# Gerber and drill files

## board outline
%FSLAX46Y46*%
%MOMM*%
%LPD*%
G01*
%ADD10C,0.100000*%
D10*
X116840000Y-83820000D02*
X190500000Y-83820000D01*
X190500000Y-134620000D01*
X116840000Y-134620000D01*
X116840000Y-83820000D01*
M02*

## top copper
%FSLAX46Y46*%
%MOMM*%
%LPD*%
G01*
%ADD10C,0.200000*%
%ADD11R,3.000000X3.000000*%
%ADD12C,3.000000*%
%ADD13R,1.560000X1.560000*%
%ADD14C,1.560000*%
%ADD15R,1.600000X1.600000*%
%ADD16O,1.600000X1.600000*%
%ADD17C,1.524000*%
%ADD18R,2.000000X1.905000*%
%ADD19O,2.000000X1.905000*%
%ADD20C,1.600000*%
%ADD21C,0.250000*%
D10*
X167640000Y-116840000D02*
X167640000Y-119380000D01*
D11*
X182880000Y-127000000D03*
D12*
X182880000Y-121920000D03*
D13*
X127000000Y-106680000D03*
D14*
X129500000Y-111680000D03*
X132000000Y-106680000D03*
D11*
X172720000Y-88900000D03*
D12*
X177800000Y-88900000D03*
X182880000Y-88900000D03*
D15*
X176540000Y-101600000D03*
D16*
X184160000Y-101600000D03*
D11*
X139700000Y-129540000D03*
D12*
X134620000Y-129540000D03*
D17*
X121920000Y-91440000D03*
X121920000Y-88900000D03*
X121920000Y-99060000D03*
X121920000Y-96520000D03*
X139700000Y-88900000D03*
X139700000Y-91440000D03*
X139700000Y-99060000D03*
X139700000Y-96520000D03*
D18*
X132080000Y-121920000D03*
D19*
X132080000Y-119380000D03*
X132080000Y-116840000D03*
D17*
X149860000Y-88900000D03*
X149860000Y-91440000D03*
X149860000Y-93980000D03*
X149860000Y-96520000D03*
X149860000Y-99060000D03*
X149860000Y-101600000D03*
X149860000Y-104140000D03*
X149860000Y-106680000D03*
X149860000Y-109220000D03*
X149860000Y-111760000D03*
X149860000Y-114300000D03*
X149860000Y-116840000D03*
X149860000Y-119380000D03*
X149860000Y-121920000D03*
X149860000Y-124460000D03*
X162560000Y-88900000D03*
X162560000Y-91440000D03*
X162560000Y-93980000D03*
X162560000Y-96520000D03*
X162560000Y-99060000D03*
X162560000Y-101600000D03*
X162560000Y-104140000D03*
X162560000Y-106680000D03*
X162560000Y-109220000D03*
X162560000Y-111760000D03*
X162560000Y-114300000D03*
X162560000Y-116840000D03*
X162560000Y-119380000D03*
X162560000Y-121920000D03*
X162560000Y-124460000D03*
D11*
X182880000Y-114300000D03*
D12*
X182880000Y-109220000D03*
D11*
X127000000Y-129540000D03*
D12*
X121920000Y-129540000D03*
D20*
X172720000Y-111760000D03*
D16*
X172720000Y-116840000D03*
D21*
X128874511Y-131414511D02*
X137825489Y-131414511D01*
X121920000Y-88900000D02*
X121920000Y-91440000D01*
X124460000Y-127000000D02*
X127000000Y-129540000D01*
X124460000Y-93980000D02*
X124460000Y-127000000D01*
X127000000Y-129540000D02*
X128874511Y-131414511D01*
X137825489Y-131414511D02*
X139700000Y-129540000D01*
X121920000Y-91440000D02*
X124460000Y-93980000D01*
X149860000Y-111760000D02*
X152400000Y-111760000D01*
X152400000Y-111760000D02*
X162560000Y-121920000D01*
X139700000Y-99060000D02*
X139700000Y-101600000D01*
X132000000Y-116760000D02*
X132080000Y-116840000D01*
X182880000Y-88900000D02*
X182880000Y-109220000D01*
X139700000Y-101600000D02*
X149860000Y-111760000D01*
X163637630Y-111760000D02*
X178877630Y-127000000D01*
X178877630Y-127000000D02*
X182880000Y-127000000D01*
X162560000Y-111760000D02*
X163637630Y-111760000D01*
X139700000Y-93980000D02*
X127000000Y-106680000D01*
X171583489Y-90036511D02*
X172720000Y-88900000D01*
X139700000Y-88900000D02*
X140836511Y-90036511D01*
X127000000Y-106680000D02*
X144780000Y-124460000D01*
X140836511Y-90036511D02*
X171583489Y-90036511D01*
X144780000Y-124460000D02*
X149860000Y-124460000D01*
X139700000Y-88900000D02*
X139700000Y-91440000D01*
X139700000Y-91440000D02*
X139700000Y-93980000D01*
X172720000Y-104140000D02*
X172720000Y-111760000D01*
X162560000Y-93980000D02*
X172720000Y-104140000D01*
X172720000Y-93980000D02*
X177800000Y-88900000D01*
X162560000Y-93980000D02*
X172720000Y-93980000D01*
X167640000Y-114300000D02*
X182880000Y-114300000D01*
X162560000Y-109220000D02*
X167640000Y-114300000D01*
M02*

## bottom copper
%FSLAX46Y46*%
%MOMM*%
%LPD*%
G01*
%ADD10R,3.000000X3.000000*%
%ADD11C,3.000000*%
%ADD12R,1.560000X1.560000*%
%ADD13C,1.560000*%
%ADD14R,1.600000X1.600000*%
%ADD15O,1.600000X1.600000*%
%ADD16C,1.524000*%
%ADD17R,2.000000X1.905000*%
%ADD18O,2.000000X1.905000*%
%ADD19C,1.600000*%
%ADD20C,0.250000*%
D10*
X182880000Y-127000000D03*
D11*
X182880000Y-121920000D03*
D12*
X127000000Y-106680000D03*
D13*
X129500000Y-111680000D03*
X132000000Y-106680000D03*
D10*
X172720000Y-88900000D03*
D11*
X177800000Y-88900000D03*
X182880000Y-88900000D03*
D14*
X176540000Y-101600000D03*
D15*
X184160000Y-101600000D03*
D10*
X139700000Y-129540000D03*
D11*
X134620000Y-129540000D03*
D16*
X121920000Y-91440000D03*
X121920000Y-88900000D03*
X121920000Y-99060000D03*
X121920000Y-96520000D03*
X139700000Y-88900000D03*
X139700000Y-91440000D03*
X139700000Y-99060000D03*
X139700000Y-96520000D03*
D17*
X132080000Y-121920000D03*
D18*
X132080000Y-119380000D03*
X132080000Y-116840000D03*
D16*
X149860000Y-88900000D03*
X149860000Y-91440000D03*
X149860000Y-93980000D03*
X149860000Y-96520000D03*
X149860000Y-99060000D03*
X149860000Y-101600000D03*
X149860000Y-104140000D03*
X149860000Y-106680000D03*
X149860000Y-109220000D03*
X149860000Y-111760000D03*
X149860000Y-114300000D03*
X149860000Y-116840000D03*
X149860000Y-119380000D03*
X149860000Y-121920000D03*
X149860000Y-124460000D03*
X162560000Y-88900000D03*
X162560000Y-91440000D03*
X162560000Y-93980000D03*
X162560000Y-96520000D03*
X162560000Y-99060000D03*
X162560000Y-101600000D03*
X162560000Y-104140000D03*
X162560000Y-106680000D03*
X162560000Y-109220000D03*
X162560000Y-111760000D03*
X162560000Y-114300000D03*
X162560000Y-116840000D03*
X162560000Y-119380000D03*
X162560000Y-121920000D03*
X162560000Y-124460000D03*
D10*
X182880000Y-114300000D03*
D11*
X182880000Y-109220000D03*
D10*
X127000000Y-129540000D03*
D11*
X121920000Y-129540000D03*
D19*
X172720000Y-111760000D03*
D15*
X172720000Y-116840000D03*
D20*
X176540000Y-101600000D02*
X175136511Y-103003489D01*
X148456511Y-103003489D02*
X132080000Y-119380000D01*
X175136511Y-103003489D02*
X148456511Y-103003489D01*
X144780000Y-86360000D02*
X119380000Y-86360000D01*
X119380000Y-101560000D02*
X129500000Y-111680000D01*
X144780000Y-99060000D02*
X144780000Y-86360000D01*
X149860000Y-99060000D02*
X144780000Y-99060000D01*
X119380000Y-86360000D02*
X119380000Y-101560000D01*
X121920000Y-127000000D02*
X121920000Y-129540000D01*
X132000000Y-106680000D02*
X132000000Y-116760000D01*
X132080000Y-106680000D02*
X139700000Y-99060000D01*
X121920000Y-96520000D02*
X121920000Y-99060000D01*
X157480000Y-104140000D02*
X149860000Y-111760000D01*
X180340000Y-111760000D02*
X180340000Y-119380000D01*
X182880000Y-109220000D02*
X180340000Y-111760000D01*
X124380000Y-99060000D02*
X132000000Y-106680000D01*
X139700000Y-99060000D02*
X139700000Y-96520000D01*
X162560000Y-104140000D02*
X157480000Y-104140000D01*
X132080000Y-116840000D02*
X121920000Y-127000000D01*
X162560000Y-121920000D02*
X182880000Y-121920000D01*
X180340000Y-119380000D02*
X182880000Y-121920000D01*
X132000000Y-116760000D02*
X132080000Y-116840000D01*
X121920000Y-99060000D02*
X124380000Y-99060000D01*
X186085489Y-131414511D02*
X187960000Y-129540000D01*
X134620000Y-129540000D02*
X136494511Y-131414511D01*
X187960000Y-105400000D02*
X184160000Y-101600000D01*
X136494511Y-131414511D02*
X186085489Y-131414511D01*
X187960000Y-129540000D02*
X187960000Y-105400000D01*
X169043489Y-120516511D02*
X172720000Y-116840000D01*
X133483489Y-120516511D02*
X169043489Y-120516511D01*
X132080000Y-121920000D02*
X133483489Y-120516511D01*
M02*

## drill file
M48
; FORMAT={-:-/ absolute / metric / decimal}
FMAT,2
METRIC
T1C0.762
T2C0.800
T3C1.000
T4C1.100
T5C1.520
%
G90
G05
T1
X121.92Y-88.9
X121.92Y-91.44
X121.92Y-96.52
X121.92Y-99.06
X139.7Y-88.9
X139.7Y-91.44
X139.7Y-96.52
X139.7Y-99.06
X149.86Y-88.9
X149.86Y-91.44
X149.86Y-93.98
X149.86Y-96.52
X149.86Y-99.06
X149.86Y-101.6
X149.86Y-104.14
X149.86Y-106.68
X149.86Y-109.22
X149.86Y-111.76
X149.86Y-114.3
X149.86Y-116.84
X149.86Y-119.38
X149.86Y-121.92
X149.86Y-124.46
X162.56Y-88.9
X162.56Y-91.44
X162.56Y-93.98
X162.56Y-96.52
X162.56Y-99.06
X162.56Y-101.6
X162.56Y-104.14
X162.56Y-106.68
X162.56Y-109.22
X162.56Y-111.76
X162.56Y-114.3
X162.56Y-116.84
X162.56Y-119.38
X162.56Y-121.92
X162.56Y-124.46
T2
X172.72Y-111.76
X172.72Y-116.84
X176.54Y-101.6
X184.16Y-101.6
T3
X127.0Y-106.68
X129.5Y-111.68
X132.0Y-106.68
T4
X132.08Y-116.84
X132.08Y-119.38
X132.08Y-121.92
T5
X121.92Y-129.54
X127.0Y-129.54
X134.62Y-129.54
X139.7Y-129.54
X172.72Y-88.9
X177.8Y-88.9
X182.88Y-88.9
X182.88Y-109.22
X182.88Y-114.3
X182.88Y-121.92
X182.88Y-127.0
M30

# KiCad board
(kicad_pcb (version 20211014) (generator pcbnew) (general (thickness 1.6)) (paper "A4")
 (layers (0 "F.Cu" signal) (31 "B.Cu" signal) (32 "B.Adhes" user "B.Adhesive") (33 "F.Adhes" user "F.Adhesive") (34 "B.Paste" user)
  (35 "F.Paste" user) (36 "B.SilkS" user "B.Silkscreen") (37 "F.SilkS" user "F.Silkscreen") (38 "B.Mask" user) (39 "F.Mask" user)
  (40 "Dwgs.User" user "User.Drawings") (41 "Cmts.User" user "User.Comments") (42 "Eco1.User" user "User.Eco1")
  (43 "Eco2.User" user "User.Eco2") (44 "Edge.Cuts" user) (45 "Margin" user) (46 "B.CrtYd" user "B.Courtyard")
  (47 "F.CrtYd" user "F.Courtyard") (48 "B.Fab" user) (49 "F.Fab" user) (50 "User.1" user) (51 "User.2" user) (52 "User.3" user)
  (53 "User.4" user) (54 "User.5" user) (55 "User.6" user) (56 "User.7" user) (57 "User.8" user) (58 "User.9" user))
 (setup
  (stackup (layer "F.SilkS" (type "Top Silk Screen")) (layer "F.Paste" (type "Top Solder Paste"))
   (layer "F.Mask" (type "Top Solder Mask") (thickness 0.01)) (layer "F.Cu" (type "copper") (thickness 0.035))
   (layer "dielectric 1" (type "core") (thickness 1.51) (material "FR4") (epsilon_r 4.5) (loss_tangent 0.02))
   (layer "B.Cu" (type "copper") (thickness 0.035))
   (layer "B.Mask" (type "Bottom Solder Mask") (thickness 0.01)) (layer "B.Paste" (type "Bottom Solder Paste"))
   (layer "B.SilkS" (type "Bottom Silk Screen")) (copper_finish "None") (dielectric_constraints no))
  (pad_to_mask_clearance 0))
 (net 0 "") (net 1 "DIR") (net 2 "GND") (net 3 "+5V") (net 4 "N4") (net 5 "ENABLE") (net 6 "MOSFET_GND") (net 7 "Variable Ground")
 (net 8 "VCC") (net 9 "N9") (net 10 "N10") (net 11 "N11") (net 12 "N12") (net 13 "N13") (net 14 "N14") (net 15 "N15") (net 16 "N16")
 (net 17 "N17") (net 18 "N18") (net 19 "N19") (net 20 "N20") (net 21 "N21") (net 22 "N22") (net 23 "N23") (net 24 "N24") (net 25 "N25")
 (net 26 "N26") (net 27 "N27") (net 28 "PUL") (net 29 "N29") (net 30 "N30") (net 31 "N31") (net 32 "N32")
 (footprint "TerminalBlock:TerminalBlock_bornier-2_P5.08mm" (layer "F.Cu") (at 182.88 127 90)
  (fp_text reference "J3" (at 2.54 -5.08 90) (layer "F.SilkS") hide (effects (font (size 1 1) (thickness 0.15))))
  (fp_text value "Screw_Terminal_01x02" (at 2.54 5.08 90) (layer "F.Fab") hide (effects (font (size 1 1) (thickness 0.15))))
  (pad "1" thru_hole rect (at 0 0 90) (size 3 3) (drill 1.52) (layers *.Cu *.Mask) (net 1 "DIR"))
  (pad "2" thru_hole circle (at 5.08 0 90) (size 3 3) (drill 1.52) (layers *.Cu *.Mask) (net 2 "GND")))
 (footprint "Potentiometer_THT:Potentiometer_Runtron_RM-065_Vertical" (layer "F.Cu") (at 127 106.68)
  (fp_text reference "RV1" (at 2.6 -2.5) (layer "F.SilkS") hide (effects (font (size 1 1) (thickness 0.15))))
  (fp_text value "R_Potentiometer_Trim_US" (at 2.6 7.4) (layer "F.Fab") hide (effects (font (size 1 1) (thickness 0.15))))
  (pad "1" thru_hole rect (at 0 0) (size 1.56 1.56) (drill 1) (layers *.Cu *.Mask) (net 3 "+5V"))
  (pad "2" thru_hole circle (at 2.5 5) (size 1.56 1.56) (drill 1) (layers *.Cu *.Mask) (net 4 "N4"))
  (pad "3" thru_hole circle (at 5 0) (size 1.56 1.56) (drill 1) (layers *.Cu *.Mask) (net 2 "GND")))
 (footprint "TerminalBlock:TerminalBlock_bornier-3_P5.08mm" (layer "F.Cu") (at 172.72 88.9)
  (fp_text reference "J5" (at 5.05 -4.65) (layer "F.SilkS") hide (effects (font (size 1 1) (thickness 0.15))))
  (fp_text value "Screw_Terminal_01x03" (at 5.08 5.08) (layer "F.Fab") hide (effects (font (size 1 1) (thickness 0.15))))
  (pad "1" thru_hole rect (at 0 0) (size 3 3) (drill 1.52) (layers *.Cu *.Mask) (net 3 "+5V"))
  (pad "2" thru_hole circle (at 5.08 0) (size 3 3) (drill 1.52) (layers *.Cu *.Mask) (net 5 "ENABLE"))
  (pad "3" thru_hole circle (at 10.16 0) (size 3 3) (drill 1.52) (layers *.Cu *.Mask) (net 2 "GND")))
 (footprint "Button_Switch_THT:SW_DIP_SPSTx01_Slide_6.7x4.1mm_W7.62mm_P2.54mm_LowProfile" (layer "F.Cu") (at 176.54 101.6)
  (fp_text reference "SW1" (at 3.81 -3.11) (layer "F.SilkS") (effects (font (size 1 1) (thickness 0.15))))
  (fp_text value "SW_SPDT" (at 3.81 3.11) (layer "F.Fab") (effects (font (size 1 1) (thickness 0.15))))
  (pad "1" thru_hole rect (at 0 0) (size 1.6 1.6) (drill 0.8) (layers *.Cu *.Mask) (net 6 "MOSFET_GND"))
  (pad "2" thru_hole oval (at 7.62 0) (size 1.6 1.6) (drill 0.8) (layers *.Cu *.Mask) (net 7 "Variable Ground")))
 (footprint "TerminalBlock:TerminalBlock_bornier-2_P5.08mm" (layer "F.Cu") (at 139.7 129.54 180)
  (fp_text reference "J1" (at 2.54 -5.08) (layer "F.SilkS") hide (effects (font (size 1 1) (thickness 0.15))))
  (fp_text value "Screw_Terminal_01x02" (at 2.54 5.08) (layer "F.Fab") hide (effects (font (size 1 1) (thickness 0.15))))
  (pad "1" thru_hole rect (at 0 0 180) (size 3 3) (drill 1.52) (layers *.Cu *.Mask) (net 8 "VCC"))
  (pad "2" thru_hole circle (at 5.08 0 180) (size 3 3) (drill 1.52) (layers *.Cu *.Mask) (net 7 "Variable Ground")))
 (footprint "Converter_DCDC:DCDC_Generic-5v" (layer "F.Cu") (at 132.08 96.52)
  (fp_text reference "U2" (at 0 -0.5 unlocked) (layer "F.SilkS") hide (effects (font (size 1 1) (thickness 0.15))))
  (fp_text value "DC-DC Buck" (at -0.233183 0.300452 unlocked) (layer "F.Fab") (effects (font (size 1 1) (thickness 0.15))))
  (pad "1" thru_hole circle (at -10.16 -5.08) (size 1.524 1.524) (drill 0.762) (layers *.Cu *.Mask) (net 8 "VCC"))
  (pad "1" thru_hole circle (at -10.16 -7.62) (size 1.524 1.524) (drill 0.762) (layers *.Cu *.Mask) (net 8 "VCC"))
  (pad "2" thru_hole circle (at -10.16 2.54) (size 1.524 1.524) (drill 0.762) (layers *.Cu *.Mask) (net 2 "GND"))
  (pad "2" thru_hole circle (at -10.16 0) (size 1.524 1.524) (drill 0.762) (layers *.Cu *.Mask) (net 2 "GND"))
  (pad "3" thru_hole circle (at 7.62 -7.62) (size 1.524 1.524) (drill 0.762) (layers *.Cu *.Mask) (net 3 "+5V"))
  (pad "3" thru_hole circle (at 7.62 -5.08) (size 1.524 1.524) (drill 0.762) (layers *.Cu *.Mask) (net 3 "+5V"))
  (pad "4" thru_hole circle (at 7.62 2.54) (size 1.524 1.524) (drill 0.762) (layers *.Cu *.Mask) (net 2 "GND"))
  (pad "4" thru_hole circle (at 7.62 0) (size 1.524 1.524) (drill 0.762) (layers *.Cu *.Mask) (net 2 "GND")))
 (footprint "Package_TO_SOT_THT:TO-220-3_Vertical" (layer "F.Cu") (at 132.08 121.92 90)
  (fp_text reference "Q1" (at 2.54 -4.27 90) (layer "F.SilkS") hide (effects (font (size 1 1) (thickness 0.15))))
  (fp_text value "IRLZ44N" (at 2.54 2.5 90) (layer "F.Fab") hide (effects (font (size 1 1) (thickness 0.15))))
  (pad "1" thru_hole rect (at 0 0 90) (size 1.905 2) (drill 1.1) (layers *.Cu *.Mask) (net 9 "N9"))
  (pad "2" thru_hole oval (at 2.54 0 90) (size 1.905 2) (drill 1.1) (layers *.Cu *.Mask) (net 6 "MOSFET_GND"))
  (pad "3" thru_hole oval (at 5.08 0 90) (size 1.905 2) (drill 1.1) (layers *.Cu *.Mask) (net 2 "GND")))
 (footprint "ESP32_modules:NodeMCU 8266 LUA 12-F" (layer "F.Cu") (at 154.94 99.06)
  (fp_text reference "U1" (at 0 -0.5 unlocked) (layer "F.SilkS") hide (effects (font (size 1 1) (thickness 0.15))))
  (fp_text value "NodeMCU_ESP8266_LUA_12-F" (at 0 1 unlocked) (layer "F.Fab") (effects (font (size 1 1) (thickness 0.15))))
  (pad "1" thru_hole circle (at -5.08 -10.16) (size 1.524 1.524) (drill 0.762) (layers *.Cu *.Mask) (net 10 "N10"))
  (pad "2" thru_hole circle (at -5.08 -7.62) (size 1.524 1.524) (drill 0.762) (layers *.Cu *.Mask) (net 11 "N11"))
  (pad "3" thru_hole circle (at -5.08 -5.08) (size 1.524 1.524) (drill 0.762) (layers *.Cu *.Mask) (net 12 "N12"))
  (pad "4" thru_hole circle (at -5.08 -2.54) (size 1.524 1.524) (drill 0.762) (layers *.Cu *.Mask) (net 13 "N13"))
  (pad "5" thru_hole circle (at -5.08 0) (size 1.524 1.524) (drill 0.762) (layers *.Cu *.Mask) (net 4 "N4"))
  (pad "6" thru_hole circle (at -5.08 2.54) (size 1.524 1.524) (drill 0.762) (layers *.Cu *.Mask) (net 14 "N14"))
  (pad "7" thru_hole circle (at -5.08 5.08) (size 1.524 1.524) (drill 0.762) (layers *.Cu *.Mask) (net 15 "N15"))
  (pad "8" thru_hole circle (at -5.08 7.62) (size 1.524 1.524) (drill 0.762) (layers *.Cu *.Mask) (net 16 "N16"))
  (pad "9" thru_hole circle (at -5.08 10.16) (size 1.524 1.524) (drill 0.762) (layers *.Cu *.Mask) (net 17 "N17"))
  (pad "10" thru_hole circle (at -5.08 12.7) (size 1.524 1.524) (drill 0.762) (layers *.Cu *.Mask) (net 2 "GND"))
  (pad "11" thru_hole circle (at -5.08 15.24) (size 1.524 1.524) (drill 0.762) (layers *.Cu *.Mask) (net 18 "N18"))
  (pad "12" thru_hole circle (at -5.08 17.78) (size 1.524 1.524) (drill 0.762) (layers *.Cu *.Mask) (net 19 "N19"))
  (pad "13" thru_hole circle (at -5.08 20.32) (size 1.524 1.524) (drill 0.762) (layers *.Cu *.Mask) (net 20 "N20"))
  (pad "14" thru_hole circle (at -5.08 22.86) (size 1.524 1.524) (drill 0.762) (layers *.Cu *.Mask) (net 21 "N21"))
  (pad "15" thru_hole circle (at -5.08 25.4) (size 1.524 1.524) (drill 0.762) (layers *.Cu *.Mask) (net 3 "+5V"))
  (pad "16" thru_hole circle (at 7.62 -10.16) (size 1.524 1.524) (drill 0.762) (layers *.Cu *.Mask) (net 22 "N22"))
  (pad "17" thru_hole circle (at 7.62 -7.62) (size 1.524 1.524) (drill 0.762) (layers *.Cu *.Mask) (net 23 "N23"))
  (pad "18" thru_hole circle (at 7.62 -5.08) (size 1.524 1.524) (drill 0.762) (layers *.Cu *.Mask) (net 5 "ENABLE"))
  (pad "19" thru_hole circle (at 7.62 -2.54) (size 1.524 1.524) (drill 0.762) (layers *.Cu *.Mask) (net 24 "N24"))
  (pad "20" thru_hole circle (at 7.62 0) (size 1.524 1.524) (drill 0.762) (layers *.Cu *.Mask) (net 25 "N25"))
  (pad "21" thru_hole circle (at 7.62 2.54) (size 1.524 1.524) (drill 0.762) (layers *.Cu *.Mask) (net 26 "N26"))
  (pad "22" thru_hole circle (at 7.62 5.08) (size 1.524 1.524) (drill 0.762) (layers *.Cu *.Mask) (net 2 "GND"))
  (pad "23" thru_hole circle (at 7.62 7.62) (size 1.524 1.524) (drill 0.762) (layers *.Cu *.Mask) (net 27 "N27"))
  (pad "24" thru_hole circle (at 7.62 10.16) (size 1.524 1.524) (drill 0.762) (layers *.Cu *.Mask) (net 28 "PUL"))
  (pad "25" thru_hole circle (at 7.62 12.7) (size 1.524 1.524) (drill 0.762) (layers *.Cu *.Mask) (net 1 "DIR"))
  (pad "26" thru_hole circle (at 7.62 15.24) (size 1.524 1.524) (drill 0.762) (layers *.Cu *.Mask) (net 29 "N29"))
  (pad "27" thru_hole circle (at 7.62 17.78) (size 1.524 1.524) (drill 0.762) (layers *.Cu *.Mask) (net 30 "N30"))
  (pad "28" thru_hole circle (at 7.62 20.32) (size 1.524 1.524) (drill 0.762) (layers *.Cu *.Mask) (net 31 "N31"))
  (pad "29" thru_hole circle (at 7.62 22.86) (size 1.524 1.524) (drill 0.762) (layers *.Cu *.Mask) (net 2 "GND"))
  (pad "30" thru_hole circle (at 7.62 25.4) (size 1.524 1.524) (drill 0.762) (layers *.Cu *.Mask) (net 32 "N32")))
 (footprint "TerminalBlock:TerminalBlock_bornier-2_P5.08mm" (layer "F.Cu") (at 182.88 114.3 90)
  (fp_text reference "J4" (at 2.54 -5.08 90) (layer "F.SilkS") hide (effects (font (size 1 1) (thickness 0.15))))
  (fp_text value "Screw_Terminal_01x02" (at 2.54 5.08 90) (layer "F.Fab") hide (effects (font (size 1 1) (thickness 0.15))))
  (pad "1" thru_hole rect (at 0 0 90) (size 3 3) (drill 1.52) (layers *.Cu *.Mask) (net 28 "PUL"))
  (pad "2" thru_hole circle (at 5.08 0 90) (size 3 3) (drill 1.52) (layers *.Cu *.Mask) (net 2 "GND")))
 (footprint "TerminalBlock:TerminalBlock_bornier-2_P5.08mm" (layer "F.Cu") (at 127 129.54 180)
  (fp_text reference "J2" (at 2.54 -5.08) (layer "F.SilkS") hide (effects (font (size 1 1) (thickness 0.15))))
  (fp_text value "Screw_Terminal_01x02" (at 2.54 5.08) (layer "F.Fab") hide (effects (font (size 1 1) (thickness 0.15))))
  (pad "1" thru_hole rect (at 0 0 180) (size 3 3) (drill 1.52) (layers *.Cu *.Mask) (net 8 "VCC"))
  (pad "2" thru_hole circle (at 5.08 0 180) (size 3 3) (drill 1.52) (layers *.Cu *.Mask) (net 2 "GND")))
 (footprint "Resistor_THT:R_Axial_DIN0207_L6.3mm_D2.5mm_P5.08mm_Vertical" (layer "F.Cu") (at 172.72 111.76 -90)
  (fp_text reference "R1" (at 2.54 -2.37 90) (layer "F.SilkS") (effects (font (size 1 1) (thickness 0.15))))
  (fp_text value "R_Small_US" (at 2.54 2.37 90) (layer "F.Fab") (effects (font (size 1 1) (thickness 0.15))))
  (pad "1" thru_hole circle (at 0 0 270) (size 1.6 1.6) (drill 0.8) (layers *.Cu *.Mask) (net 5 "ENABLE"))
  (pad "2" thru_hole oval (at 5.08 0 270) (size 1.6 1.6) (drill 0.8) (layers *.Cu *.Mask) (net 9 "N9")))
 (gr_line (start 167.64 116.84) (end 167.64 119.38) (layer "F.Cu") (width 0.2))
 (gr_rect (start 116.84 83.82) (end 190.5 134.62) (layer "Edge.Cuts") (width 0.1) (fill none))
 (segment (start 128.874511 131.414511) (end 137.825489 131.414511) (width 0.25) (layer "F.Cu") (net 8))
 (segment (start 121.92 88.9) (end 121.92 91.44) (width 0.25) (layer "F.Cu") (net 8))
 (segment (start 124.46 127) (end 127 129.54) (width 0.25) (layer "F.Cu") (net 8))
 (segment (start 124.46 93.98) (end 124.46 127) (width 0.25) (layer "F.Cu") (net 8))
 (segment (start 127 129.54) (end 128.874511 131.414511) (width 0.25) (layer "F.Cu") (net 8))
 (segment (start 137.825489 131.414511) (end 139.7 129.54) (width 0.25) (layer "F.Cu") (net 8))
 (segment (start 121.92 91.44) (end 124.46 93.98) (width 0.25) (layer "F.Cu") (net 8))
 (segment (start 176.54 101.6) (end 175.136511 103.003489) (width 0.25) (layer "B.Cu") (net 6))
 (segment (start 148.456511 103.003489) (end 132.08 119.38) (width 0.25) (layer "B.Cu") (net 6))
 (segment (start 175.136511 103.003489) (end 148.456511 103.003489) (width 0.25) (layer "B.Cu") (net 6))
 (segment (start 144.78 86.36) (end 119.38 86.36) (width 0.25) (layer "B.Cu") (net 4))
 (segment (start 119.38 101.56) (end 129.5 111.68) (width 0.25) (layer "B.Cu") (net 4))
 (segment (start 144.78 99.06) (end 144.78 86.36) (width 0.25) (layer "B.Cu") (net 4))
 (segment (start 149.86 99.06) (end 144.78 99.06) (width 0.25) (layer "B.Cu") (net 4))
 (segment (start 119.38 86.36) (end 119.38 101.56) (width 0.25) (layer "B.Cu") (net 4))
 (segment (start 149.86 111.76) (end 152.4 111.76) (width 0.25) (layer "F.Cu") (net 2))
 (segment (start 152.4 111.76) (end 162.56 121.92) (width 0.25) (layer "F.Cu") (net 2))
 (segment (start 139.7 99.06) (end 139.7 101.6) (width 0.25) (layer "F.Cu") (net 2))
 (segment (start 132 116.76) (end 132.08 116.84) (width 0.25) (layer "F.Cu") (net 2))
 (segment (start 182.88 88.9) (end 182.88 109.22) (width 0.25) (layer "F.Cu") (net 2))
 (segment (start 139.7 101.6) (end 149.86 111.76) (width 0.25) (layer "F.Cu") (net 2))
 (segment (start 121.92 127) (end 121.92 129.54) (width 0.25) (layer "B.Cu") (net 2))
 (segment (start 132 106.68) (end 132 116.76) (width 0.25) (layer "B.Cu") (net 2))
 (segment (start 132.08 106.68) (end 139.7 99.06) (width 0.25) (layer "B.Cu") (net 2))
 (segment (start 121.92 96.52) (end 121.92 99.06) (width 0.25) (layer "B.Cu") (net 2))
 (segment (start 157.48 104.14) (end 149.86 111.76) (width 0.25) (layer "B.Cu") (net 2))
 (segment (start 180.34 111.76) (end 180.34 119.38) (width 0.25) (layer "B.Cu") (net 2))
 (segment (start 182.88 109.22) (end 180.34 111.76) (width 0.25) (layer "B.Cu") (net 2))
 (segment (start 124.38 99.06) (end 132 106.68) (width 0.25) (layer "B.Cu") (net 2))
 (segment (start 139.7 99.06) (end 139.7 96.52) (width 0.25) (layer "B.Cu") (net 2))
 (segment (start 162.56 104.14) (end 157.48 104.14) (width 0.25) (layer "B.Cu") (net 2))
 (segment (start 132.08 116.84) (end 121.92 127) (width 0.25) (layer "B.Cu") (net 2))
 (segment (start 162.56 121.92) (end 182.88 121.92) (width 0.25) (layer "B.Cu") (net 2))
 (segment (start 180.34 119.38) (end 182.88 121.92) (width 0.25) (layer "B.Cu") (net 2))
 (segment (start 132 116.76) (end 132.08 116.84) (width 0.25) (layer "B.Cu") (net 2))
 (segment (start 121.92 99.06) (end 124.38 99.06) (width 0.25) (layer "B.Cu") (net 2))
 (segment (start 186.085489 131.414511) (end 187.96 129.54) (width 0.25) (layer "B.Cu") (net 7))
 (segment (start 134.62 129.54) (end 136.494511 131.414511) (width 0.25) (layer "B.Cu") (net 7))
 (segment (start 187.96 105.4) (end 184.16 101.6) (width 0.25) (layer "B.Cu") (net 7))
 (segment (start 136.494511 131.414511) (end 186.085489 131.414511) (width 0.25) (layer "B.Cu") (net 7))
 (segment (start 187.96 129.54) (end 187.96 105.4) (width 0.25) (layer "B.Cu") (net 7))
 (segment (start 163.63763 111.76) (end 178.87763 127) (width 0.25) (layer "F.Cu") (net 1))
 (segment (start 178.87763 127) (end 182.88 127) (width 0.25) (layer "F.Cu") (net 1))
 (segment (start 162.56 111.76) (end 163.63763 111.76) (width 0.25) (layer "F.Cu") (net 1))
 (segment (start 139.7 93.98) (end 127 106.68) (width 0.25) (layer "F.Cu") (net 3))
 (segment (start 171.583489 90.036511) (end 172.72 88.9) (width 0.25) (layer "F.Cu") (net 3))
 (segment (start 139.7 88.9) (end 140.836511 90.036511) (width 0.25) (layer "F.Cu") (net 3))
 (segment (start 127 106.68) (end 144.78 124.46) (width 0.25) (layer "F.Cu") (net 3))
 (segment (start 140.836511 90.036511) (end 171.583489 90.036511) (width 0.25) (layer "F.Cu") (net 3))
 (segment (start 144.78 124.46) (end 149.86 124.46) (width 0.25) (layer "F.Cu") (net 3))
 (segment (start 139.7 88.9) (end 139.7 91.44) (width 0.25) (layer "F.Cu") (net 3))
 (segment (start 139.7 91.44) (end 139.7 93.98) (width 0.25) (layer "F.Cu") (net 3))
 (segment (start 172.72 104.14) (end 172.72 111.76) (width 0.25) (layer "F.Cu") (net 5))
 (segment (start 162.56 93.98) (end 172.72 104.14) (width 0.25) (layer "F.Cu") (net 5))
 (segment (start 172.72 93.98) (end 177.8 88.9) (width 0.25) (layer "F.Cu") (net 5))
 (segment (start 162.56 93.98) (end 172.72 93.98) (width 0.25) (layer "F.Cu") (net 5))
 (segment (start 167.64 114.3) (end 182.88 114.3) (width 0.25) (layer "F.Cu") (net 28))
 (segment (start 162.56 109.22) (end 167.64 114.3) (width 0.25) (layer "F.Cu") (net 28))
 (segment (start 169.043489 120.516511) (end 172.72 116.84) (width 0.25) (layer "B.Cu") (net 9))
 (segment (start 133.483489 120.516511) (end 169.043489 120.516511) (width 0.25) (layer "B.Cu") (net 9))
 (segment (start 132.08 121.92) (end 133.483489 120.516511) (width 0.25) (layer "B.Cu") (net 9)))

